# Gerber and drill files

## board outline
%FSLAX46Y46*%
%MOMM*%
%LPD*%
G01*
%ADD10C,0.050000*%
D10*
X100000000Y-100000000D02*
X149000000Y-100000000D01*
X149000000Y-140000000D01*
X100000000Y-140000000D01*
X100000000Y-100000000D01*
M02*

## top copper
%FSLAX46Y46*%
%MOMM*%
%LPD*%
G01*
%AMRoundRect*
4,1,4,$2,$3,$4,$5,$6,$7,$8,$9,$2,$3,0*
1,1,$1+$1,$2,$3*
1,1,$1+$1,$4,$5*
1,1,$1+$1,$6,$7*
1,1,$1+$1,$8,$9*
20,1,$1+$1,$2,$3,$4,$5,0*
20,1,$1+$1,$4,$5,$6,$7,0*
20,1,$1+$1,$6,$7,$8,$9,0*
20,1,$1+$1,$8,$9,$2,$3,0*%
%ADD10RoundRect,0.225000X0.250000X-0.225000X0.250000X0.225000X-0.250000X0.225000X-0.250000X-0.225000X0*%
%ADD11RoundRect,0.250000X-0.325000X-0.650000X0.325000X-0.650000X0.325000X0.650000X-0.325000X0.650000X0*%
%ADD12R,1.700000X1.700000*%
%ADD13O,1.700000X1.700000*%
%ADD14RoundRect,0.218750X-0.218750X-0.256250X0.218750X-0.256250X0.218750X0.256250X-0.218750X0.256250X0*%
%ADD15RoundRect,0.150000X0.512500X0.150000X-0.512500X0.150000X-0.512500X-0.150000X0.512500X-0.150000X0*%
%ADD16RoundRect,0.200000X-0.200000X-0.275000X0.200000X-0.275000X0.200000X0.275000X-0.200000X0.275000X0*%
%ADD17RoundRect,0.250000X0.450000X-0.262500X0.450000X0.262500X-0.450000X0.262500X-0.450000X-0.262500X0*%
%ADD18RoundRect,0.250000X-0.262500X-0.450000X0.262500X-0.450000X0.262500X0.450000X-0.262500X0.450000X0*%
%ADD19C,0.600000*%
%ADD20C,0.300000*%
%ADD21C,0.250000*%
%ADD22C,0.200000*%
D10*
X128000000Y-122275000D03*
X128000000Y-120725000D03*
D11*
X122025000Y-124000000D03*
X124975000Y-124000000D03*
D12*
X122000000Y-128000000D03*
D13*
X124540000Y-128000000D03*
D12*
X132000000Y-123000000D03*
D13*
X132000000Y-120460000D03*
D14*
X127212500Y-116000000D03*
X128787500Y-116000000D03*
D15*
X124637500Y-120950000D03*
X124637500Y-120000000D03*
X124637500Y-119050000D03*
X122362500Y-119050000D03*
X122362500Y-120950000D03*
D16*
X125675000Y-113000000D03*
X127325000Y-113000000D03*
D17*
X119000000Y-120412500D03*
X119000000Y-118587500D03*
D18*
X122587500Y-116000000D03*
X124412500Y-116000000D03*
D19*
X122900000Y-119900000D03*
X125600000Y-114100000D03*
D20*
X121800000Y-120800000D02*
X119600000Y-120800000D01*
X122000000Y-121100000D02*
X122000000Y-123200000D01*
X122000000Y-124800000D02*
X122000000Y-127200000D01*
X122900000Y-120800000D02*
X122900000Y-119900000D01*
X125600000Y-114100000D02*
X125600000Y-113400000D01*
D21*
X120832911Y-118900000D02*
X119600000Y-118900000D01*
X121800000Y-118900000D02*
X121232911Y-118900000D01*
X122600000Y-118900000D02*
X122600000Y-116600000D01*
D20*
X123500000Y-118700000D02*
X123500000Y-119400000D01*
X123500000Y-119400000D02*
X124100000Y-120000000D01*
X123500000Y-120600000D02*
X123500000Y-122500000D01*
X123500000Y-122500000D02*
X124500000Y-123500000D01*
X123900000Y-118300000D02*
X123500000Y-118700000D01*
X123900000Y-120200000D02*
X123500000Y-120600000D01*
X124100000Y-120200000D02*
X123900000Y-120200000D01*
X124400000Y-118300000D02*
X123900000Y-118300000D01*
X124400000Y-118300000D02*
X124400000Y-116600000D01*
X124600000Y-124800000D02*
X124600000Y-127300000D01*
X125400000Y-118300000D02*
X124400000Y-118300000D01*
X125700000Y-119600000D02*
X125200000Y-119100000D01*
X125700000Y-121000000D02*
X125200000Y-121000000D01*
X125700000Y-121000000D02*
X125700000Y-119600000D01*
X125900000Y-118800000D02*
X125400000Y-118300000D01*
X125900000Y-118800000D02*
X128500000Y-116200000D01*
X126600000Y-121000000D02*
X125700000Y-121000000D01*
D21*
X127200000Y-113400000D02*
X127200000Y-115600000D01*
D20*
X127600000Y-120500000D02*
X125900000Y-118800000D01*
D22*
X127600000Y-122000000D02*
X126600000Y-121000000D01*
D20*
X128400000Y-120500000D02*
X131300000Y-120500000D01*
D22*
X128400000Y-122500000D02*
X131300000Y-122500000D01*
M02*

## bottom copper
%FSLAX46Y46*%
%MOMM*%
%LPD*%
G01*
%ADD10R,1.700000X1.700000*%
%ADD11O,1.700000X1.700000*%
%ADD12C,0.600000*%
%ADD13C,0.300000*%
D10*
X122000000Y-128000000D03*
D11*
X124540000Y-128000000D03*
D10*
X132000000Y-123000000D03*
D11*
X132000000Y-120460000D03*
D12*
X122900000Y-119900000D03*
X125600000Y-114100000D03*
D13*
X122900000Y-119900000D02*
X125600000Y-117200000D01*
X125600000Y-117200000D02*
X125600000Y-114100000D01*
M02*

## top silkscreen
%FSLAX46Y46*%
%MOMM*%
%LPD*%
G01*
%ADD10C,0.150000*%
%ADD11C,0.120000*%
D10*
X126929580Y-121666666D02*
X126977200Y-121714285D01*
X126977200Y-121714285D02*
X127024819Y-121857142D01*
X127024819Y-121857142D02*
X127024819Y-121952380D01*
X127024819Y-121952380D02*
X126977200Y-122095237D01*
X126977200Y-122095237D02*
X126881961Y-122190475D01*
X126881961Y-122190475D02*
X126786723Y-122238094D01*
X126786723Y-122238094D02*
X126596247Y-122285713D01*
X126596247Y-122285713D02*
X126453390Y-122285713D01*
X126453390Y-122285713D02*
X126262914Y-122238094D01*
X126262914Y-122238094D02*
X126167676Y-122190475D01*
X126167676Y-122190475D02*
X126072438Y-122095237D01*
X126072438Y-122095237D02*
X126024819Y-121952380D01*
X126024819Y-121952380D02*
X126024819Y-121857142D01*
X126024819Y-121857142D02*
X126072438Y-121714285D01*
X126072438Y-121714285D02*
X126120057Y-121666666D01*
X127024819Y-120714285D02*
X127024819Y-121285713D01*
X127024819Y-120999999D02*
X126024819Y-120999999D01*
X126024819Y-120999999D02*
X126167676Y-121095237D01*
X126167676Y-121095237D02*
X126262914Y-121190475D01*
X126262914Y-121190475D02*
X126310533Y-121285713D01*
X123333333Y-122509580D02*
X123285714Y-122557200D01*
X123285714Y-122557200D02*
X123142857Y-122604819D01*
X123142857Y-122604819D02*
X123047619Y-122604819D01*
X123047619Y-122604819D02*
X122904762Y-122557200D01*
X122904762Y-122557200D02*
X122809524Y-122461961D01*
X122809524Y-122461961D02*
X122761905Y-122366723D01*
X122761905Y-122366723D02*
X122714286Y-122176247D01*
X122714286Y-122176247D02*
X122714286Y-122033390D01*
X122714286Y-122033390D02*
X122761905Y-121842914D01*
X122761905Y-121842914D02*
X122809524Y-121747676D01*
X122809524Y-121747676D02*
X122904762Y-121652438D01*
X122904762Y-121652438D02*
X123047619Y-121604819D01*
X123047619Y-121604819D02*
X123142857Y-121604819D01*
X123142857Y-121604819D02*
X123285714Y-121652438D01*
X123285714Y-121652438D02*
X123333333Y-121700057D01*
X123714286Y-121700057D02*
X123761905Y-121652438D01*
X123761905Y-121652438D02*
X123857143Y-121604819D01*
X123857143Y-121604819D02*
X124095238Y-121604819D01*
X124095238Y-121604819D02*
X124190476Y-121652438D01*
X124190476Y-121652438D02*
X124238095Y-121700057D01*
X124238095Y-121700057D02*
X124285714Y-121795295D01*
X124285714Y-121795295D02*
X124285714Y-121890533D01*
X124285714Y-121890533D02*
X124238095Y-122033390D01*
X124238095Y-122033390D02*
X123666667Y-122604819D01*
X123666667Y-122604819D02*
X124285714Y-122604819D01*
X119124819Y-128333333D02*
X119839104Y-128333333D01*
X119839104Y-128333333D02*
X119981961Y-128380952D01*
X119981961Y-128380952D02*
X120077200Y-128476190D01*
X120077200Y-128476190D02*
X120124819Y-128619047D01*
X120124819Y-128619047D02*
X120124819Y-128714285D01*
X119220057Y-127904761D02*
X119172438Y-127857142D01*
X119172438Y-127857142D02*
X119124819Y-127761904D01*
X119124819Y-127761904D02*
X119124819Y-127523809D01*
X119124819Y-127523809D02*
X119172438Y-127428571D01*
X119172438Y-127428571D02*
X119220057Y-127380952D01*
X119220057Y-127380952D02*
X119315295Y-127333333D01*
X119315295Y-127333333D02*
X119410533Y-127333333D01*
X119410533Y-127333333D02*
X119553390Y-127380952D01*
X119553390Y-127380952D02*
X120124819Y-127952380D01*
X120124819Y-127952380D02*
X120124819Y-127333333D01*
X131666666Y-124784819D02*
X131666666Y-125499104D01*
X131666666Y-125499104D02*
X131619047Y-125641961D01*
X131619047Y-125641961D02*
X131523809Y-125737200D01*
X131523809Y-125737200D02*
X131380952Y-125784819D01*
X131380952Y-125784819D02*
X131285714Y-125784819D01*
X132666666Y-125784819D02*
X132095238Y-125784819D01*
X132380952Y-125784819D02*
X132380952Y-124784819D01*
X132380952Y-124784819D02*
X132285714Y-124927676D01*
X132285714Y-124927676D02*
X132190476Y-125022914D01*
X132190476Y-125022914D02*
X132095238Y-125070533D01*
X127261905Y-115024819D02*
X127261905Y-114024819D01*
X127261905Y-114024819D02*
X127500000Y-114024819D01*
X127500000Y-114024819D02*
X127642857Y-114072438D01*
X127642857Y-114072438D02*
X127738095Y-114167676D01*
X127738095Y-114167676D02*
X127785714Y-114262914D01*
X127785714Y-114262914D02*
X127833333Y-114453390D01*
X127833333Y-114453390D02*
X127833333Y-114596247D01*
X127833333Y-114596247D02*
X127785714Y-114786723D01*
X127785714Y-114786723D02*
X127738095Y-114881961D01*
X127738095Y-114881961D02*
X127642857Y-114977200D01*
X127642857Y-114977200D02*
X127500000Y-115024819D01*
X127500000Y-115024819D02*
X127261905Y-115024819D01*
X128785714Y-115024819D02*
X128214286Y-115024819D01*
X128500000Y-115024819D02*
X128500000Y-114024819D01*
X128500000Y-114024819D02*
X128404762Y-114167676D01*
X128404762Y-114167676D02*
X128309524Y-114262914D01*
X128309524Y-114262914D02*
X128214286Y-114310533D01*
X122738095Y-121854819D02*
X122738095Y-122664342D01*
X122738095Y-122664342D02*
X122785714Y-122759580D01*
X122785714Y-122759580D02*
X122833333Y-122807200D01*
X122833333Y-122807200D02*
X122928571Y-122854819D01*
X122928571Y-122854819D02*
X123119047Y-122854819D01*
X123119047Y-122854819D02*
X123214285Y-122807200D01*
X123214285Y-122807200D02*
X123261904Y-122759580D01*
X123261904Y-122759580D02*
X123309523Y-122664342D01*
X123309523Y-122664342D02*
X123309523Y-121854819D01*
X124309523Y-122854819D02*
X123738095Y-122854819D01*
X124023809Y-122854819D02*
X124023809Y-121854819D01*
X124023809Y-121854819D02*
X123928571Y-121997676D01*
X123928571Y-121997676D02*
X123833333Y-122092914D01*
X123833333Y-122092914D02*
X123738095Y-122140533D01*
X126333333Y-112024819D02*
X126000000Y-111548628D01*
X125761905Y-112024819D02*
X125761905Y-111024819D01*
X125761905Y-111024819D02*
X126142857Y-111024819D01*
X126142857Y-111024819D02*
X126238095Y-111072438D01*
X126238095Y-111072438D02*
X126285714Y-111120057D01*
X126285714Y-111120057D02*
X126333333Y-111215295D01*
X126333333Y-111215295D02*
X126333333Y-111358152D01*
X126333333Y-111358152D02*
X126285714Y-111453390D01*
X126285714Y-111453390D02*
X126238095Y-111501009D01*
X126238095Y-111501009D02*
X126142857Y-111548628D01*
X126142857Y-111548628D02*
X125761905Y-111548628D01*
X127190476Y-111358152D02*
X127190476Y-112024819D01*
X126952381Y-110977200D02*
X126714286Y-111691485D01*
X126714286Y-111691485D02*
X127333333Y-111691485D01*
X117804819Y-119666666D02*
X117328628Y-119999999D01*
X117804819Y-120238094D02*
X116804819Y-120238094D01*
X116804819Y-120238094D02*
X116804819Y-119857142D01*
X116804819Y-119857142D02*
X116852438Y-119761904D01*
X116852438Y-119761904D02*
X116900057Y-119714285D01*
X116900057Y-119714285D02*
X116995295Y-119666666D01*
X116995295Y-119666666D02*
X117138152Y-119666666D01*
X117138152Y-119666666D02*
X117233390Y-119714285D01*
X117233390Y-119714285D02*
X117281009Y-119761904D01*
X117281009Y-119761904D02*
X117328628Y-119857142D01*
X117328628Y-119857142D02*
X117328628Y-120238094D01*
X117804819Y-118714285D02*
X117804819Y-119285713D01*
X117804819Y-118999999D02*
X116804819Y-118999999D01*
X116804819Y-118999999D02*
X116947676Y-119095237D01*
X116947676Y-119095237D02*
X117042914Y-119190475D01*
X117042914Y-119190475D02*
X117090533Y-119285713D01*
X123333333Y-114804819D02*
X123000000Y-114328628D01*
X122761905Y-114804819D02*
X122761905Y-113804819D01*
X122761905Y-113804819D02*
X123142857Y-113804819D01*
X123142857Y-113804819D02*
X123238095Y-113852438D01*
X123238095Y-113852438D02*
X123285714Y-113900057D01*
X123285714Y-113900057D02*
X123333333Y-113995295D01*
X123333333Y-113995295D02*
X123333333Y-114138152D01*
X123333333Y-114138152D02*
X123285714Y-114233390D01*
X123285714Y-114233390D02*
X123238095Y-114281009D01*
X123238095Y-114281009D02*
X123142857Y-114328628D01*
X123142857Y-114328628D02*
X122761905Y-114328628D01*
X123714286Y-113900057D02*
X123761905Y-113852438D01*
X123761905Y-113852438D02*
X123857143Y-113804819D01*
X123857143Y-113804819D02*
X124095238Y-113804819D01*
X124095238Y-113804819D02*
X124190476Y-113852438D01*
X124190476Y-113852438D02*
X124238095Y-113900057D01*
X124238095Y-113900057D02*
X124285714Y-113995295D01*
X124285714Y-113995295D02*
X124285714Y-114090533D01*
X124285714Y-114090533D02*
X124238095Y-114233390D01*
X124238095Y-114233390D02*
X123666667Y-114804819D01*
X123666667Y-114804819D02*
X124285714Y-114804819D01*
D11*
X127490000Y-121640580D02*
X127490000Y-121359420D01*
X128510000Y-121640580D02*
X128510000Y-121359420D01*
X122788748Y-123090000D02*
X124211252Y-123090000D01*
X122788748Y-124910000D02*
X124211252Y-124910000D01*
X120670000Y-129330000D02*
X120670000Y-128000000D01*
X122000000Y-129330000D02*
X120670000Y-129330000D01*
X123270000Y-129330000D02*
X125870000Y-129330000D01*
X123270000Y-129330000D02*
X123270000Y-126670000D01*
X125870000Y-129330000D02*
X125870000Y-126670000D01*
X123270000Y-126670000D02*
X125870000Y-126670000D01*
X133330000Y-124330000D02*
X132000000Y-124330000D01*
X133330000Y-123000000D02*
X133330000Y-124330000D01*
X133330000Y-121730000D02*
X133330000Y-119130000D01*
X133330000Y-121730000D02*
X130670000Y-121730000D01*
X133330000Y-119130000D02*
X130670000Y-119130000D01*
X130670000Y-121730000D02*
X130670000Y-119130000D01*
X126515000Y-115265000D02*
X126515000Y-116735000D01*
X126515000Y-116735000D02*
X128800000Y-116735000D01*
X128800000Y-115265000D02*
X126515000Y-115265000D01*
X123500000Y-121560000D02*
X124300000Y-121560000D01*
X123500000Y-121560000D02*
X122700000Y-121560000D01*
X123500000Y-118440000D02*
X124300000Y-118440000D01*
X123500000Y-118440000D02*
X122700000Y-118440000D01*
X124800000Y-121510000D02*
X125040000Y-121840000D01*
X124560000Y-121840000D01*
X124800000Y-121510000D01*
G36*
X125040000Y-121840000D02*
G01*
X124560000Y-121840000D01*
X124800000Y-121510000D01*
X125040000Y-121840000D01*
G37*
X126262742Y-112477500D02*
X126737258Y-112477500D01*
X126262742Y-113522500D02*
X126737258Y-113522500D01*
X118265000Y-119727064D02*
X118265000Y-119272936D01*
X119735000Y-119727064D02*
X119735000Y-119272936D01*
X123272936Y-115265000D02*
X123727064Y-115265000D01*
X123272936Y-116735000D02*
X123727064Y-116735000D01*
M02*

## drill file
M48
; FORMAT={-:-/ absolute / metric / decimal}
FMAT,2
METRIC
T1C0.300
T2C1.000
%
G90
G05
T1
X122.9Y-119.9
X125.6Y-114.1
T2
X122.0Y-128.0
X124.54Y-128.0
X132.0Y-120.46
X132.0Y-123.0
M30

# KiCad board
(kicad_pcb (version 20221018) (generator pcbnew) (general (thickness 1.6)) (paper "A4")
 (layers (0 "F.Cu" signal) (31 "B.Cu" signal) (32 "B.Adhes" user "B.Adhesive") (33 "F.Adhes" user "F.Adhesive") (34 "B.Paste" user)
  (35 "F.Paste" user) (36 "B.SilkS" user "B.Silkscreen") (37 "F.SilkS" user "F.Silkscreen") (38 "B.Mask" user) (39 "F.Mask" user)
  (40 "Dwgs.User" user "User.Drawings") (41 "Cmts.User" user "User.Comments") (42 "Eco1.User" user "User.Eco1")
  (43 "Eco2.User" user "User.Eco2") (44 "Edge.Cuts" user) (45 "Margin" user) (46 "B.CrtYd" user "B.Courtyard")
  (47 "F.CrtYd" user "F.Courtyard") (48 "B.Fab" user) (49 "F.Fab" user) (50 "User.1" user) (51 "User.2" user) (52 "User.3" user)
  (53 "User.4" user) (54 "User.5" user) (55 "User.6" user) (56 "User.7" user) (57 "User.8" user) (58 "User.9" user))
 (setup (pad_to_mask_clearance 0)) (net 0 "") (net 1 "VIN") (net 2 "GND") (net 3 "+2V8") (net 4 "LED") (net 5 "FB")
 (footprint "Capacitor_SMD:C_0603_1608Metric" (layer "F.Cu") (at 128 121.5 90)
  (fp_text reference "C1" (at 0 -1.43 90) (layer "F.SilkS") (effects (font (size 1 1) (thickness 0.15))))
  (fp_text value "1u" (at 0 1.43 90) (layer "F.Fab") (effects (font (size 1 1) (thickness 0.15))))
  (fp_line (start -0.14058 -0.51) (end 0.14058 -0.51) (stroke (width 0.12) (type solid)) (layer "F.SilkS"))
  (fp_line (start -0.14058 0.51) (end 0.14058 0.51) (stroke (width 0.12) (type solid)) (layer "F.SilkS"))
  (pad "1" smd roundrect (at -0.775 0 90) (size 0.9 0.95) (layers "F.Cu" "F.Paste" "F.Mask") (roundrect_rratio 0.25) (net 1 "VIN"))
  (pad "2" smd roundrect (at 0.775 0 90) (size 0.9 0.95) (layers "F.Cu" "F.Paste" "F.Mask") (roundrect_rratio 0.25) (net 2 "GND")))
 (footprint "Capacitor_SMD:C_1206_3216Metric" (layer "F.Cu") (at 123.5 124)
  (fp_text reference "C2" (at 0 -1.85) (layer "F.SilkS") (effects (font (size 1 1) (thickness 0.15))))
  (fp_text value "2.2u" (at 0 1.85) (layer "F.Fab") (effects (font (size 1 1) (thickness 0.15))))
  (fp_line (start -0.711252 -0.91) (end 0.711252 -0.91) (stroke (width 0.12) (type solid)) (layer "F.SilkS"))
  (fp_line (start -0.711252 0.91) (end 0.711252 0.91) (stroke (width 0.12) (type solid)) (layer "F.SilkS"))
  (pad "1" smd roundrect (at -1.475 0) (size 1.15 1.8) (layers "F.Cu" "F.Paste" "F.Mask") (roundrect_rratio 0.217391) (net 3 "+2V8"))
  (pad "2" smd roundrect (at 1.475 0) (size 1.15 1.8) (layers "F.Cu" "F.Paste" "F.Mask") (roundrect_rratio 0.217391) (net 2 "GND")))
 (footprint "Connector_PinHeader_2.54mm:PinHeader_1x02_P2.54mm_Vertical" (layer "F.Cu") (at 122 128 90)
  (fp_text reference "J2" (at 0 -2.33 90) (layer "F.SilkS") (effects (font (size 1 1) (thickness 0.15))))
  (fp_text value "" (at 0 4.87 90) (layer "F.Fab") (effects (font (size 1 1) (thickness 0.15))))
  (fp_line (start -1.33 -1.33) (end 0 -1.33) (stroke (width 0.12) (type solid)) (layer "F.SilkS"))
  (fp_line (start -1.33 0) (end -1.33 -1.33) (stroke (width 0.12) (type solid)) (layer "F.SilkS"))
  (fp_line (start -1.33 1.27) (end -1.33 3.87) (stroke (width 0.12) (type solid)) (layer "F.SilkS"))
  (fp_line (start -1.33 1.27) (end 1.33 1.27) (stroke (width 0.12) (type solid)) (layer "F.SilkS"))
  (fp_line (start -1.33 3.87) (end 1.33 3.87) (stroke (width 0.12) (type solid)) (layer "F.SilkS"))
  (fp_line (start 1.33 1.27) (end 1.33 3.87) (stroke (width 0.12) (type solid)) (layer "F.SilkS"))
  (pad "1" thru_hole rect (at 0 0 90) (size 1.7 1.7) (drill 1) (layers "*.Cu" "*.Mask") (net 3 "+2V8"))
  (pad "2" thru_hole oval (at 0 2.54 90) (size 1.7 1.7) (drill 1) (layers "*.Cu" "*.Mask") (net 2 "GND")))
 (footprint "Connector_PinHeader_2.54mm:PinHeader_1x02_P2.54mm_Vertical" (layer "F.Cu") (at 132 123 180)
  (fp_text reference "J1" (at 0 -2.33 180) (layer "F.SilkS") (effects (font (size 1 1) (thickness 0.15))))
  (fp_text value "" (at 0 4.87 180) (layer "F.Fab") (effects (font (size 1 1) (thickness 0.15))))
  (fp_line (start -1.33 -1.33) (end 0 -1.33) (stroke (width 0.12) (type solid)) (layer "F.SilkS"))
  (fp_line (start -1.33 0) (end -1.33 -1.33) (stroke (width 0.12) (type solid)) (layer "F.SilkS"))
  (fp_line (start -1.33 1.27) (end -1.33 3.87) (stroke (width 0.12) (type solid)) (layer "F.SilkS"))
  (fp_line (start -1.33 1.27) (end 1.33 1.27) (stroke (width 0.12) (type solid)) (layer "F.SilkS"))
  (fp_line (start -1.33 3.87) (end 1.33 3.87) (stroke (width 0.12) (type solid)) (layer "F.SilkS"))
  (fp_line (start 1.33 1.27) (end 1.33 3.87) (stroke (width 0.12) (type solid)) (layer "F.SilkS"))
  (pad "1" thru_hole rect (at 0 0 180) (size 1.7 1.7) (drill 1) (layers "*.Cu" "*.Mask") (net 1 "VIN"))
  (pad "2" thru_hole oval (at 0 2.54 180) (size 1.7 1.7) (drill 1) (layers "*.Cu" "*.Mask") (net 2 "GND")))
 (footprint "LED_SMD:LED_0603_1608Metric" (layer "F.Cu") (at 128 116)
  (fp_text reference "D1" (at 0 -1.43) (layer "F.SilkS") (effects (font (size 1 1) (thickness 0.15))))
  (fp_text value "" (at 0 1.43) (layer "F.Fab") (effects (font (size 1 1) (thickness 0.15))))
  (fp_line (start -1.485 -0.735) (end -1.485 0.735) (stroke (width 0.12) (type solid)) (layer "F.SilkS"))
  (fp_line (start -1.485 0.735) (end 0.8 0.735) (stroke (width 0.12) (type solid)) (layer "F.SilkS"))
  (fp_line (start 0.8 -0.735) (end -1.485 -0.735) (stroke (width 0.12) (type solid)) (layer "F.SilkS"))
  (pad "1" smd roundrect (at -0.7875 0) (size 0.875 0.95) (layers "F.Cu" "F.Paste" "F.Mask") (roundrect_rratio 0.25) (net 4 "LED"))
  (pad "2" smd roundrect (at 0.7875 0) (size 0.875 0.95) (layers "F.Cu" "F.Paste" "F.Mask") (roundrect_rratio 0.25) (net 2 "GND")))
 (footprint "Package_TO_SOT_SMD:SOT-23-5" (layer "F.Cu") (at 123.5 120 180)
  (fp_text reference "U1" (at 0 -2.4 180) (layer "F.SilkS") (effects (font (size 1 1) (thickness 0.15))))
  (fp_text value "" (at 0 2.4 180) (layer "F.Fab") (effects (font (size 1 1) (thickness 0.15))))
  (fp_line (start 0 -1.56) (end -0.8 -1.56) (stroke (width 0.12) (type solid)) (layer "F.SilkS"))
  (fp_line (start 0 -1.56) (end 0.8 -1.56) (stroke (width 0.12) (type solid)) (layer "F.SilkS"))
  (fp_line (start 0 1.56) (end -0.8 1.56) (stroke (width 0.12) (type solid)) (layer "F.SilkS"))
  (fp_line (start 0 1.56) (end 0.8 1.56) (stroke (width 0.12) (type solid)) (layer "F.SilkS"))
  (fp_poly
   (pts (xy -1.3 -1.51) (xy -1.54 -1.84) (xy -1.06 -1.84) (xy -1.3 -1.51)) (stroke (width 0.12) (type solid)) (fill solid) (layer "F.SilkS"))
  (pad "1" smd roundrect (at -1.1375 -0.95 180) (size 1.325 0.6) (layers "F.Cu" "F.Paste" "F.Mask") (roundrect_rratio 0.25) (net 1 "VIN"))
  (pad "2" smd roundrect (at -1.1375 0 180) (size 1.325 0.6) (layers "F.Cu" "F.Paste" "F.Mask") (roundrect_rratio 0.25) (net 2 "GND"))
  (pad "3" smd roundrect (at -1.1375 0.95 180) (size 1.325 0.6) (layers "F.Cu" "F.Paste" "F.Mask") (roundrect_rratio 0.25) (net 1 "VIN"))
  (pad "4" smd roundrect (at 1.1375 0.95 180) (size 1.325 0.6) (layers "F.Cu" "F.Paste" "F.Mask") (roundrect_rratio 0.25) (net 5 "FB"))
  (pad "5" smd roundrect (at 1.1375 -0.95 180) (size 1.325 0.6) (layers "F.Cu" "F.Paste" "F.Mask") (roundrect_rratio 0.25) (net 3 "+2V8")))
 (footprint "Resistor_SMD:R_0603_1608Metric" (layer "F.Cu") (at 126.5 113)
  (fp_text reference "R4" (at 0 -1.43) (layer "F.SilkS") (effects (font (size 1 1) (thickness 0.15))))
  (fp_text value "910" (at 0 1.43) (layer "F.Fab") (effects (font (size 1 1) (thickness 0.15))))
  (fp_line (start -0.237258 -0.5225) (end 0.237258 -0.5225) (stroke (width 0.12) (type solid)) (layer "F.SilkS"))
  (fp_line (start -0.237258 0.5225) (end 0.237258 0.5225) (stroke (width 0.12) (type solid)) (layer "F.SilkS"))
  (pad "1" smd roundrect (at -0.825 0) (size 0.8 0.95) (layers "F.Cu" "F.Paste" "F.Mask") (roundrect_rratio 0.25) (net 3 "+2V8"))
  (pad "2" smd roundrect (at 0.825 0) (size 0.8 0.95) (layers "F.Cu" "F.Paste" "F.Mask") (roundrect_rratio 0.25) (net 4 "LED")))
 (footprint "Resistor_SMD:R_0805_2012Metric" (layer "F.Cu") (at 119 119.5 90)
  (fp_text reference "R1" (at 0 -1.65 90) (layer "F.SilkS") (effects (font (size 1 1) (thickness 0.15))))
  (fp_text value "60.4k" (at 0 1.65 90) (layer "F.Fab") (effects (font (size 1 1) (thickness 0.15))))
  (fp_line (start -0.227064 -0.735) (end 0.227064 -0.735) (stroke (width 0.12) (type solid)) (layer "F.SilkS"))
  (fp_line (start -0.227064 0.735) (end 0.227064 0.735) (stroke (width 0.12) (type solid)) (layer "F.SilkS"))
  (pad "1" smd roundrect (at -0.9125 0 90) (size 1.025 1.4) (layers "F.Cu" "F.Paste" "F.Mask") (roundrect_rratio 0.243902) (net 3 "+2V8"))
  (pad "2" smd roundrect (at 0.9125 0 90) (size 1.025 1.4) (layers "F.Cu" "F.Paste" "F.Mask") (roundrect_rratio 0.243902) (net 5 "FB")))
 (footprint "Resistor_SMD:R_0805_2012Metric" (layer "F.Cu") (at 123.5 116)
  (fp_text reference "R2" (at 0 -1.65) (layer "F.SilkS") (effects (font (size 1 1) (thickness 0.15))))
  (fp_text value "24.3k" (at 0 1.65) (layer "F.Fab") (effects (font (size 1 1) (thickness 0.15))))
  (fp_line (start -0.227064 -0.735) (end 0.227064 -0.735) (stroke (width 0.12) (type solid)) (layer "F.SilkS"))
  (fp_line (start -0.227064 0.735) (end 0.227064 0.735) (stroke (width 0.12) (type solid)) (layer "F.SilkS"))
  (pad "1" smd roundrect (at -0.9125 0) (size 1.025 1.4) (layers "F.Cu" "F.Paste" "F.Mask") (roundrect_rratio 0.243902) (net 5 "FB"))
  (pad "2" smd roundrect (at 0.9125 0) (size 1.025 1.4) (layers "F.Cu" "F.Paste" "F.Mask") (roundrect_rratio 0.243902) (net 2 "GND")))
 (gr_rect (start 100 100) (end 149 140) (stroke (width 0.05) (type default)) (fill none) (layer "Edge.Cuts"))
 (segment (start 121.8 120.8) (end 119.6 120.8) (width 0.3) (layer "F.Cu") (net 3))
 (segment (start 122 121.1) (end 122 123.2) (width 0.3) (layer "F.Cu") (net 3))
 (segment (start 122 124.8) (end 122 127.2) (width 0.3) (layer "F.Cu") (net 3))
 (segment (start 122.9 120.8) (end 122.9 119.9) (width 0.3) (layer "F.Cu") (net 3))
 (segment (start 125.6 114.1) (end 125.6 113.4) (width 0.3) (layer "F.Cu") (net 3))
 (via (at 122.9 119.9) (size 0.6) (drill 0.3) (layers "F.Cu" "B.Cu") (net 3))
 (via (at 125.6 114.1) (size 0.6) (drill 0.3) (layers "F.Cu" "B.Cu") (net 3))
 (segment (start 120.832911 118.9) (end 119.6 118.9) (width 0.25) (layer "F.Cu") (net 5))
 (segment (start 121.8 118.9) (end 121.232911 118.9) (width 0.25) (layer "F.Cu") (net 5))
 (segment (start 122.6 118.9) (end 122.6 116.6) (width 0.25) (layer "F.Cu") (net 5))
 (segment (start 122.9 119.9) (end 125.6 117.2) (width 0.3) (layer "B.Cu") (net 3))
 (segment (start 123.5 118.7) (end 123.5 119.4) (width 0.3) (layer "F.Cu") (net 2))
 (segment (start 123.5 119.4) (end 124.1 120) (width 0.3) (layer "F.Cu") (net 2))
 (segment (start 123.5 120.6) (end 123.5 122.5) (width 0.3) (layer "F.Cu") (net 2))
 (segment (start 123.5 122.5) (end 124.5 123.5) (width 0.3) (layer "F.Cu") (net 2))
 (segment (start 123.9 118.3) (end 123.5 118.7) (width 0.3) (layer "F.Cu") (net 2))
 (segment (start 123.9 120.2) (end 123.5 120.6) (width 0.3) (layer "F.Cu") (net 2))
 (segment (start 124.1 120.2) (end 123.9 120.2) (width 0.3) (layer "F.Cu") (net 2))
 (segment (start 124.4 118.3) (end 123.9 118.3) (width 0.3) (layer "F.Cu") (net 2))
 (segment (start 124.4 118.3) (end 124.4 116.6) (width 0.3) (layer "F.Cu") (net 2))
 (segment (start 124.6 124.8) (end 124.6 127.3) (width 0.3) (layer "F.Cu") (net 2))
 (segment (start 125.4 118.3) (end 124.4 118.3) (width 0.3) (layer "F.Cu") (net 2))
 (segment (start 125.6 117.2) (end 125.6 114.1) (width 0.3) (layer "B.Cu") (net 3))
 (segment (start 125.7 119.6) (end 125.2 119.1) (width 0.3) (layer "F.Cu") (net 1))
 (segment (start 125.7 121) (end 125.2 121) (width 0.3) (layer "F.Cu") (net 1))
 (segment (start 125.7 121) (end 125.7 119.6) (width 0.3) (layer "F.Cu") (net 1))
 (segment (start 125.9 118.8) (end 125.4 118.3) (width 0.3) (layer "F.Cu") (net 2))
 (segment (start 125.9 118.8) (end 128.5 116.2) (width 0.3) (layer "F.Cu") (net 2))
 (segment (start 126.6 121) (end 125.7 121) (width 0.3) (layer "F.Cu") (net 1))
 (segment (start 127.2 113.4) (end 127.2 115.6) (width 0.25) (layer "F.Cu") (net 4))
 (segment (start 127.6 120.5) (end 125.9 118.8) (width 0.3) (layer "F.Cu") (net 2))
 (segment (start 127.6 122) (end 126.6 121) (width 0.2) (layer "F.Cu") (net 1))
 (segment (start 128.4 120.5) (end 131.3 120.5) (width 0.3) (layer "F.Cu") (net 2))
 (segment (start 128.4 122.5) (end 131.3 122.5) (width 0.2) (layer "F.Cu") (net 1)))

